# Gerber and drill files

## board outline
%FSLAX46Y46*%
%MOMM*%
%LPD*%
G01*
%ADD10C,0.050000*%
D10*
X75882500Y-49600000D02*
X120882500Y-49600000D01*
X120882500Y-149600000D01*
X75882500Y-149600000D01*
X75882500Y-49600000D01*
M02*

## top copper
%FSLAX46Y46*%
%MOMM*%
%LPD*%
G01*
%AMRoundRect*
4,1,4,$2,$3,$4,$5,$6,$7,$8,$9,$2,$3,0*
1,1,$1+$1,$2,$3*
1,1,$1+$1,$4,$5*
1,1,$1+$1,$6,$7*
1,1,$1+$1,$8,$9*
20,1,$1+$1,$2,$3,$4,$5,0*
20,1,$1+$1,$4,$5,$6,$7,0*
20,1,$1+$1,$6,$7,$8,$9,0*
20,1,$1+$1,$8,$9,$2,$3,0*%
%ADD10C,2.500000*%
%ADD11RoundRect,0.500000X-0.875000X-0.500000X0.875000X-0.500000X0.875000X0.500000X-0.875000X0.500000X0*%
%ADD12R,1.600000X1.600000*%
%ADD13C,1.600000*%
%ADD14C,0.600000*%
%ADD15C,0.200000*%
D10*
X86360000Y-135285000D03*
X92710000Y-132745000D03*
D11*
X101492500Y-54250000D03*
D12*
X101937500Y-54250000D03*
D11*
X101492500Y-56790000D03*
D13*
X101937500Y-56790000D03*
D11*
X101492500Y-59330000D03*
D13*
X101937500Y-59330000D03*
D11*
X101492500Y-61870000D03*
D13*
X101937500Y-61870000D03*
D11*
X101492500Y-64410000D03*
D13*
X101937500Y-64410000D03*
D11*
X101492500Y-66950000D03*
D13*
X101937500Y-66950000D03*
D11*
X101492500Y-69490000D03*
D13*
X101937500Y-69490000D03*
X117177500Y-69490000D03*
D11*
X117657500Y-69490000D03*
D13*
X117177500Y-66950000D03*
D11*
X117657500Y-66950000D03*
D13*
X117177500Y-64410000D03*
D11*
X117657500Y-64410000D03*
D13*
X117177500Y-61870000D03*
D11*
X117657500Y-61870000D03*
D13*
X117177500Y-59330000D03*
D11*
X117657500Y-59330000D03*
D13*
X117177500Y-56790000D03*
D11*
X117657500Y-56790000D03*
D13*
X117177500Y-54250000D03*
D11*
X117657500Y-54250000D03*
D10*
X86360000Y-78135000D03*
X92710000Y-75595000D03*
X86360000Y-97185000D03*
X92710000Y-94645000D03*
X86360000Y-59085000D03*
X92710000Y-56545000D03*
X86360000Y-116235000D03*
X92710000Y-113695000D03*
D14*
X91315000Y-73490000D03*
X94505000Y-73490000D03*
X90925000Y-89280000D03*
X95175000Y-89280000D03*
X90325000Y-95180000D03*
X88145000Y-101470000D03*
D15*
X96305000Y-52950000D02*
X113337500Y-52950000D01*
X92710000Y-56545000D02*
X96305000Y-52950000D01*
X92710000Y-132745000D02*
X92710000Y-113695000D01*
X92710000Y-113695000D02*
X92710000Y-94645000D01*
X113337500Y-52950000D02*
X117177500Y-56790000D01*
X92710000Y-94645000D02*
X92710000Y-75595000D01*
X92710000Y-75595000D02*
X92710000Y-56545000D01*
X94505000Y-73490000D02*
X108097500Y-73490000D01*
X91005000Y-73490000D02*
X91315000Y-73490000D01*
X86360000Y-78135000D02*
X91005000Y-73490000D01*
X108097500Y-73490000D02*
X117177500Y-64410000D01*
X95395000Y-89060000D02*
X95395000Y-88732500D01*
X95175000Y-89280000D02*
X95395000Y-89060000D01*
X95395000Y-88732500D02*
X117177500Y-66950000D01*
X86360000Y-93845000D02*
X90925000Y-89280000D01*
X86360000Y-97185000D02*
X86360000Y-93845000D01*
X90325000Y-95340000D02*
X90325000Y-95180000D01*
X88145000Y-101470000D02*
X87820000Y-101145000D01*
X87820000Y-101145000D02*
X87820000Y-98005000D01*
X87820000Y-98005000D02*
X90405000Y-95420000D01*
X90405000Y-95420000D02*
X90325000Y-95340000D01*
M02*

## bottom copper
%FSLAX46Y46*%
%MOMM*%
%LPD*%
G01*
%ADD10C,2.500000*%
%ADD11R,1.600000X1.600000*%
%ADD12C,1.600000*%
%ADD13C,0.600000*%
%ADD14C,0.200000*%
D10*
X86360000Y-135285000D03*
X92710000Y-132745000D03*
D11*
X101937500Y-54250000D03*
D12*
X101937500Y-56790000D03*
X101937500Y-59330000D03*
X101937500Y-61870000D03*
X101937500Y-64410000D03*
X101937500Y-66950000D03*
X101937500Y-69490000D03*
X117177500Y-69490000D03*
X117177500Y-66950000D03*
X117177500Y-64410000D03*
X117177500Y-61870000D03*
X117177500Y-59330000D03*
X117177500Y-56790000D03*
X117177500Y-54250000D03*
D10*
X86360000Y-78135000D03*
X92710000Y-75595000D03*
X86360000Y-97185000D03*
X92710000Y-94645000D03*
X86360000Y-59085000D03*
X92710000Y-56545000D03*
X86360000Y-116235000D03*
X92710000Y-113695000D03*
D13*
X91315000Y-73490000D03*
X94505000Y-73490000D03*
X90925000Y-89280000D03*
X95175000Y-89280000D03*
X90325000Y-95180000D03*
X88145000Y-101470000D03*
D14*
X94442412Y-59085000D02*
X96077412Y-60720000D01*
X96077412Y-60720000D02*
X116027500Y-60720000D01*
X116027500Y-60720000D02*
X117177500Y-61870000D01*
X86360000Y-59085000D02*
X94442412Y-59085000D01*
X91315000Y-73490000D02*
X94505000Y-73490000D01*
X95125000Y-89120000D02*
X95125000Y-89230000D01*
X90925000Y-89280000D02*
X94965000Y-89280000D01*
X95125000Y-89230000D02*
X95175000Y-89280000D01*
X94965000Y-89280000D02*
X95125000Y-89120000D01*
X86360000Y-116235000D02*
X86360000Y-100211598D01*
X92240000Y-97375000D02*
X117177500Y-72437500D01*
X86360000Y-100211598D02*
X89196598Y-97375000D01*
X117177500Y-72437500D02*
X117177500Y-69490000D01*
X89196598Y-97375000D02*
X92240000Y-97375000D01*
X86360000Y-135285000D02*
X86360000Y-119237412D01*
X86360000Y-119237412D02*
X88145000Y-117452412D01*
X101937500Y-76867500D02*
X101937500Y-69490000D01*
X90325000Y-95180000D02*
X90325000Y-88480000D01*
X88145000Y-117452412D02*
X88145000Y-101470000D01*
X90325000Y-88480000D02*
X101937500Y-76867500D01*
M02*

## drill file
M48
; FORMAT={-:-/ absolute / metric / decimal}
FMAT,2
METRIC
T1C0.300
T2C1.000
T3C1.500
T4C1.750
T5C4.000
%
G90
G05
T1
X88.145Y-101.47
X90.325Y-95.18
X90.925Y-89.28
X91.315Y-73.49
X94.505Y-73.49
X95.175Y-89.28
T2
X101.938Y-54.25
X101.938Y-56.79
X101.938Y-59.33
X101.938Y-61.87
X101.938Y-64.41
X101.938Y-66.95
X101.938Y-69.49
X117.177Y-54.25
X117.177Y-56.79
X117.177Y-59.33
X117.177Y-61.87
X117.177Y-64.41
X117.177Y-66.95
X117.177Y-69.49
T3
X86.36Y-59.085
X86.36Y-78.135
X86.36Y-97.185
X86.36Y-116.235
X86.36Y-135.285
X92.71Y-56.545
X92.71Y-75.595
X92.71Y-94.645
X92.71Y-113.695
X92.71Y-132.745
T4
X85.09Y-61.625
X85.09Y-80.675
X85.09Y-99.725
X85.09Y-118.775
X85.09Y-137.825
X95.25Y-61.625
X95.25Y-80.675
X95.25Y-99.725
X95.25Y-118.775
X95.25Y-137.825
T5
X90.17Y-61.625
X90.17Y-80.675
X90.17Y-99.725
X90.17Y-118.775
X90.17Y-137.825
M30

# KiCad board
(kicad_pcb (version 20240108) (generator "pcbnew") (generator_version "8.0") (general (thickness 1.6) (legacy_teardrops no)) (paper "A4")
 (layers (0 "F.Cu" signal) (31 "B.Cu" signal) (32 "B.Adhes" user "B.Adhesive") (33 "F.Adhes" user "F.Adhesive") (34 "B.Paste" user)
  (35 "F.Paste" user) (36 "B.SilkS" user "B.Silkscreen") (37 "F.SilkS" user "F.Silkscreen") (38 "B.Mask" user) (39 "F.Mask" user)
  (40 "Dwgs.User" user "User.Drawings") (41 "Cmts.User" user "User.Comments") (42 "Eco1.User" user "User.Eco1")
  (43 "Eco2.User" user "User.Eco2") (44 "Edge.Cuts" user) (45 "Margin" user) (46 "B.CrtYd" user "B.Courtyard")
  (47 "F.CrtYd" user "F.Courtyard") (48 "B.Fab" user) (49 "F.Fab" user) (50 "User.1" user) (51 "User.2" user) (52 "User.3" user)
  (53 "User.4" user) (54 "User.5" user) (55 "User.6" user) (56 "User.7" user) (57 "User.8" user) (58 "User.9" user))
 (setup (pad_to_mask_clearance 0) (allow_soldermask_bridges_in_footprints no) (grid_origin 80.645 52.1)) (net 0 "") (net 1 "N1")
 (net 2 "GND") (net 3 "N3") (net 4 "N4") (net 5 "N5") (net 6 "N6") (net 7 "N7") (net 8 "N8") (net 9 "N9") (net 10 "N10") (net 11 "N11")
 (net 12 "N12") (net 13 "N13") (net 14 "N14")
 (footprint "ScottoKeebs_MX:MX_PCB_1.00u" (layer "F.Cu") (at 90.17 137.825)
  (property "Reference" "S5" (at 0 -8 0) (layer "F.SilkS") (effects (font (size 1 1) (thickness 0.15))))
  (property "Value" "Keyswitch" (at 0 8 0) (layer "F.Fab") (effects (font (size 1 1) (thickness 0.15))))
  (pad "" np_thru_hole circle (at -5.08 0) (size 1.75 1.75) (drill 1.75) (layers "*.Cu" "*.Mask"))
  (pad "" np_thru_hole circle (at 0 0) (size 4 4) (drill 4) (layers "*.Cu" "*.Mask"))
  (pad "" np_thru_hole circle (at 5.08 0) (size 1.75 1.75) (drill 1.75) (layers "*.Cu" "*.Mask"))
  (pad "1" thru_hole circle (at -3.81 -2.54) (size 2.5 2.5) (drill 1.5) (layers "*.Cu" "*.Mask") (remove_unused_layers no) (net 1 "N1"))
  (pad "2" thru_hole circle (at 2.54 -5.08) (size 2.5 2.5) (drill 1.5) (layers "*.Cu" "*.Mask") (remove_unused_layers no) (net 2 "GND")))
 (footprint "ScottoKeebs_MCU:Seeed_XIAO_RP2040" (layer "F.Cu") (at 109.5575 61.87)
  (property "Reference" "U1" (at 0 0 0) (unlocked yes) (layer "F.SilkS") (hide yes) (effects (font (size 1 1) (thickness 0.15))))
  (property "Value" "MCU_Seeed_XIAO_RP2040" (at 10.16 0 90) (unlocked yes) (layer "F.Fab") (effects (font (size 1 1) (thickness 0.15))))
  (pad "1" smd roundrect (at -8.065 -7.62) (size 2.75 2) (layers "F.Cu" "F.Paste" "F.Mask") (roundrect_rratio 0.25) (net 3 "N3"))
  (pad "1" thru_hole rect (at -7.62 -7.62 90) (size 1.6 1.6) (drill 1) (layers "*.Cu" "*.Mask") (remove_unused_layers no) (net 3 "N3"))
  (pad "2" smd roundrect (at -8.065 -5.08) (size 2.75 2) (layers "F.Cu" "F.Paste" "F.Mask") (roundrect_rratio 0.25) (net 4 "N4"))
  (pad "2" thru_hole circle (at -7.62 -5.08 90) (size 1.6 1.6) (drill 1) (layers "*.Cu" "*.Mask") (remove_unused_layers no) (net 4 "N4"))
  (pad "3" smd roundrect (at -8.065 -2.54) (size 2.75 2) (layers "F.Cu" "F.Paste" "F.Mask") (roundrect_rratio 0.25) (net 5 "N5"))
  (pad "3" thru_hole circle (at -7.62 -2.54 90) (size 1.6 1.6) (drill 1) (layers "*.Cu" "*.Mask") (remove_unused_layers no) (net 5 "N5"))
  (pad "4" smd roundrect (at -8.065 0) (size 2.75 2) (layers "F.Cu" "F.Paste" "F.Mask") (roundrect_rratio 0.25) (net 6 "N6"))
  (pad "4" thru_hole circle (at -7.62 0 90) (size 1.6 1.6) (drill 1) (layers "*.Cu" "*.Mask") (remove_unused_layers no) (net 6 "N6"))
  (pad "5" smd roundrect (at -8.065 2.54) (size 2.75 2) (layers "F.Cu" "F.Paste" "F.Mask") (roundrect_rratio 0.25) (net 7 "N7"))
  (pad "5" thru_hole circle (at -7.62 2.54 90) (size 1.6 1.6) (drill 1) (layers "*.Cu" "*.Mask") (remove_unused_layers no) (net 7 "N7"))
  (pad "6" smd roundrect (at -8.065 5.08) (size 2.75 2) (layers "F.Cu" "F.Paste" "F.Mask") (roundrect_rratio 0.25) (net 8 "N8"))
  (pad "6" thru_hole circle (at -7.62 5.08 90) (size 1.6 1.6) (drill 1) (layers "*.Cu" "*.Mask") (remove_unused_layers no) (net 8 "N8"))
  (pad "7" smd roundrect (at -8.065 7.62) (size 2.75 2) (layers "F.Cu" "F.Paste" "F.Mask") (roundrect_rratio 0.25) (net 1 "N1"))
  (pad "7" thru_hole circle (at -7.62 7.62 90) (size 1.6 1.6) (drill 1) (layers "*.Cu" "*.Mask") (remove_unused_layers no) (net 1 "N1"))
  (pad "8" thru_hole circle (at 7.62 7.62 90) (size 1.6 1.6) (drill 1) (layers "*.Cu" "*.Mask") (remove_unused_layers no) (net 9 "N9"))
  (pad "8" smd roundrect (at 8.1 7.62) (size 2.75 2) (layers "F.Cu" "F.Paste" "F.Mask") (roundrect_rratio 0.25) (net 9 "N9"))
  (pad "9" thru_hole circle (at 7.62 5.08 90) (size 1.6 1.6) (drill 1) (layers "*.Cu" "*.Mask") (remove_unused_layers no) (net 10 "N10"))
  (pad "9" smd roundrect (at 8.1 5.08) (size 2.75 2) (layers "F.Cu" "F.Paste" "F.Mask") (roundrect_rratio 0.25) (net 10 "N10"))
  (pad "10" thru_hole circle (at 7.62 2.54 90) (size 1.6 1.6) (drill 1) (layers "*.Cu" "*.Mask") (remove_unused_layers no) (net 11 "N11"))
  (pad "10" smd roundrect (at 8.1 2.54) (size 2.75 2) (layers "F.Cu" "F.Paste" "F.Mask") (roundrect_rratio 0.25) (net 11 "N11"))
  (pad "11" thru_hole circle (at 7.62 0 90) (size 1.6 1.6) (drill 1) (layers "*.Cu" "*.Mask") (remove_unused_layers no) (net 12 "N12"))
  (pad "11" smd roundrect (at 8.1 0) (size 2.75 2) (layers "F.Cu" "F.Paste" "F.Mask") (roundrect_rratio 0.25) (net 12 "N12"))
  (pad "12" thru_hole circle (at 7.62 -2.54 90) (size 1.6 1.6) (drill 1) (layers "*.Cu" "*.Mask") (remove_unused_layers no) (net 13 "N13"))
  (pad "12" smd roundrect (at 8.1 -2.54) (size 2.75 2) (layers "F.Cu" "F.Paste" "F.Mask") (roundrect_rratio 0.25) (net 13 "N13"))
  (pad "13" thru_hole circle (at 7.62 -5.08 90) (size 1.6 1.6) (drill 1) (layers "*.Cu" "*.Mask") (remove_unused_layers no) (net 2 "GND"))
  (pad "13" smd roundrect (at 8.1 -5.08) (size 2.75 2) (layers "F.Cu" "F.Paste" "F.Mask") (roundrect_rratio 0.25) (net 2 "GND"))
  (pad "14" thru_hole circle (at 7.62 -7.62 90) (size 1.6 1.6) (drill 1) (layers "*.Cu" "*.Mask") (remove_unused_layers no) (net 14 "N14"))
  (pad "14" smd roundrect (at 8.1 -7.62) (size 2.75 2) (layers "F.Cu" "F.Paste" "F.Mask") (roundrect_rratio 0.25) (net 14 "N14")))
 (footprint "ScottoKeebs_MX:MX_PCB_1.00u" (layer "F.Cu") (at 90.17 80.675)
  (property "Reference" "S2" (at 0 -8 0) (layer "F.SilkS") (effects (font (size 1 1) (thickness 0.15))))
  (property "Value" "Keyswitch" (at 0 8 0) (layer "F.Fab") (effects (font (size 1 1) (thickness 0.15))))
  (pad "" np_thru_hole circle (at -5.08 0) (size 1.75 1.75) (drill 1.75) (layers "*.Cu" "*.Mask"))
  (pad "" np_thru_hole circle (at 0 0) (size 4 4) (drill 4) (layers "*.Cu" "*.Mask"))
  (pad "" np_thru_hole circle (at 5.08 0) (size 1.75 1.75) (drill 1.75) (layers "*.Cu" "*.Mask"))
  (pad "1" thru_hole circle (at -3.81 -2.54) (size 2.5 2.5) (drill 1.5) (layers "*.Cu" "*.Mask") (remove_unused_layers no) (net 11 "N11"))
  (pad "2" thru_hole circle (at 2.54 -5.08) (size 2.5 2.5) (drill 1.5) (layers "*.Cu" "*.Mask") (remove_unused_layers no) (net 2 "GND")))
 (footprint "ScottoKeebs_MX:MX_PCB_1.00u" (layer "F.Cu") (at 90.17 99.725)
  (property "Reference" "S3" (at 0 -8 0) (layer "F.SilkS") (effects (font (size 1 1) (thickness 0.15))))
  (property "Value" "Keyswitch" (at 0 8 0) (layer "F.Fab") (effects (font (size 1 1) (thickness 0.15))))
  (pad "" np_thru_hole circle (at -5.08 0) (size 1.75 1.75) (drill 1.75) (layers "*.Cu" "*.Mask"))
  (pad "" np_thru_hole circle (at 0 0) (size 4 4) (drill 4) (layers "*.Cu" "*.Mask"))
  (pad "" np_thru_hole circle (at 5.08 0) (size 1.75 1.75) (drill 1.75) (layers "*.Cu" "*.Mask"))
  (pad "1" thru_hole circle (at -3.81 -2.54) (size 2.5 2.5) (drill 1.5) (layers "*.Cu" "*.Mask") (remove_unused_layers no) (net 10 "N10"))
  (pad "2" thru_hole circle (at 2.54 -5.08) (size 2.5 2.5) (drill 1.5) (layers "*.Cu" "*.Mask") (remove_unused_layers no) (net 2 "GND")))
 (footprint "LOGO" (layer "F.Cu") (at 116.71771 92.292004 -90)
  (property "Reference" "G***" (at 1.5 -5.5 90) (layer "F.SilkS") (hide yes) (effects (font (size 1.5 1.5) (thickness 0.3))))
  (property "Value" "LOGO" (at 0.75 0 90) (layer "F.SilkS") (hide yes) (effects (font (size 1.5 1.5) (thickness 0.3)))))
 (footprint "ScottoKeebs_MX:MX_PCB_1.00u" (layer "F.Cu") (at 90.17 61.625)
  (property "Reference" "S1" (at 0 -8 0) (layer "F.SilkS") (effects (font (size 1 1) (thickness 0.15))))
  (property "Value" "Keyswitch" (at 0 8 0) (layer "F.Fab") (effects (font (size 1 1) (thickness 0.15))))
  (pad "" np_thru_hole circle (at -5.08 0) (size 1.75 1.75) (drill 1.75) (layers "*.Cu" "*.Mask"))
  (pad "" np_thru_hole circle (at 0 0) (size 4 4) (drill 4) (layers "*.Cu" "*.Mask"))
  (pad "" np_thru_hole circle (at 5.08 0) (size 1.75 1.75) (drill 1.75) (layers "*.Cu" "*.Mask"))
  (pad "1" thru_hole circle (at -3.81 -2.54) (size 2.5 2.5) (drill 1.5) (layers "*.Cu" "*.Mask") (remove_unused_layers no) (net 12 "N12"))
  (pad "2" thru_hole circle (at 2.54 -5.08) (size 2.5 2.5) (drill 1.5) (layers "*.Cu" "*.Mask") (remove_unused_layers no) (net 2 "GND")))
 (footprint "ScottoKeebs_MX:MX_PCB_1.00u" (layer "F.Cu") (at 90.17 118.775)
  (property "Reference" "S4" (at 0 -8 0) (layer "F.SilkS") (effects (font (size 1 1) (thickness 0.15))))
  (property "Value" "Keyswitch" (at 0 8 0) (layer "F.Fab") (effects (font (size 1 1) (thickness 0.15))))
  (pad "" np_thru_hole circle (at -5.08 0) (size 1.75 1.75) (drill 1.75) (layers "*.Cu" "*.Mask"))
  (pad "" np_thru_hole circle (at 0 0) (size 4 4) (drill 4) (layers "*.Cu" "*.Mask"))
  (pad "" np_thru_hole circle (at 5.08 0) (size 1.75 1.75) (drill 1.75) (layers "*.Cu" "*.Mask"))
  (pad "1" thru_hole circle (at -3.81 -2.54) (size 2.5 2.5) (drill 1.5) (layers "*.Cu" "*.Mask") (remove_unused_layers no) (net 9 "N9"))
  (pad "2" thru_hole circle (at 2.54 -5.08) (size 2.5 2.5) (drill 1.5) (layers "*.Cu" "*.Mask") (remove_unused_layers no) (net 2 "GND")))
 (gr_rect (start 75.8825 49.6) (end 120.8825 149.6) (stroke (width 0.05) (type default)) (fill none) (layer "Edge.Cuts"))
 (segment (start 96.305 52.95) (end 113.3375 52.95) (width 0.2) (layer "F.Cu") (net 2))
 (segment (start 92.71 56.545) (end 96.305 52.95) (width 0.2) (layer "F.Cu") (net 2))
 (segment (start 92.71 132.745) (end 92.71 113.695) (width 0.2) (layer "F.Cu") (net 2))
 (segment (start 92.71 113.695) (end 92.71 94.645) (width 0.2) (layer "F.Cu") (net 2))
 (segment (start 113.3375 52.95) (end 117.1775 56.79) (width 0.2) (layer "F.Cu") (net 2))
 (segment (start 92.71 94.645) (end 92.71 75.595) (width 0.2) (layer "F.Cu") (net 2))
 (segment (start 92.71 75.595) (end 92.71 56.545) (width 0.2) (layer "F.Cu") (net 2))
 (segment (start 94.442412 59.085) (end 96.077412 60.72) (width 0.2) (layer "B.Cu") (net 12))
 (segment (start 96.077412 60.72) (end 116.0275 60.72) (width 0.2) (layer "B.Cu") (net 12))
 (segment (start 116.0275 60.72) (end 117.1775 61.87) (width 0.2) (layer "B.Cu") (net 12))
 (segment (start 86.36 59.085) (end 94.442412 59.085) (width 0.2) (layer "B.Cu") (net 12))
 (segment (start 94.505 73.49) (end 108.0975 73.49) (width 0.2) (layer "F.Cu") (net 11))
 (segment (start 91.005 73.49) (end 91.315 73.49) (width 0.2) (layer "F.Cu") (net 11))
 (segment (start 86.36 78.135) (end 91.005 73.49) (width 0.2) (layer "F.Cu") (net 11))
 (segment (start 108.0975 73.49) (end 117.1775 64.41) (width 0.2) (layer "F.Cu") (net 11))
 (via (at 91.315 73.49) (size 0.6) (drill 0.3) (layers "F.Cu" "B.Cu") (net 11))
 (via (at 94.505 73.49) (size 0.6) (drill 0.3) (layers "F.Cu" "B.Cu") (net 11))
 (segment (start 91.315 73.49) (end 94.505 73.49) (width 0.2) (layer "B.Cu") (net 11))
 (segment (start 95.395 89.06) (end 95.395 88.7325) (width 0.2) (layer "F.Cu") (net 10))
 (segment (start 95.175 89.28) (end 95.395 89.06) (width 0.2) (layer "F.Cu") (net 10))
 (segment (start 95.395 88.7325) (end 117.1775 66.95) (width 0.2) (layer "F.Cu") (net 10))
 (segment (start 86.36 93.845) (end 90.925 89.28) (width 0.2) (layer "F.Cu") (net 10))
 (segment (start 86.36 97.185) (end 86.36 93.845) (width 0.2) (layer "F.Cu") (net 10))
 (via (at 90.925 89.28) (size 0.6) (drill 0.3) (layers "F.Cu" "B.Cu") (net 10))
 (via (at 95.175 89.28) (size 0.6) (drill 0.3) (layers "F.Cu" "B.Cu") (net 10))
 (segment (start 95.125 89.12) (end 95.125 89.23) (width 0.2) (layer "B.Cu") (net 10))
 (segment (start 90.925 89.28) (end 94.965 89.28) (width 0.2) (layer "B.Cu") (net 10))
 (segment (start 95.125 89.23) (end 95.175 89.28) (width 0.2) (layer "B.Cu") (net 10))
 (segment (start 94.965 89.28) (end 95.125 89.12) (width 0.2) (layer "B.Cu") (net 10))
 (segment (start 86.36 116.235) (end 86.36 100.211598) (width 0.2) (layer "B.Cu") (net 9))
 (segment (start 92.24 97.375) (end 117.1775 72.4375) (width 0.2) (layer "B.Cu") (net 9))
 (segment (start 86.36 100.211598) (end 89.196598 97.375) (width 0.2) (layer "B.Cu") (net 9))
 (segment (start 117.1775 72.4375) (end 117.1775 69.49) (width 0.2) (layer "B.Cu") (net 9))
 (segment (start 89.196598 97.375) (end 92.24 97.375) (width 0.2) (layer "B.Cu") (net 9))
 (segment (start 90.325 95.34) (end 90.325 95.18) (width 0.2) (layer "F.Cu") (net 1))
 (segment (start 88.145 101.47) (end 87.82 101.145) (width 0.2) (layer "F.Cu") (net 1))
 (segment (start 87.82 101.145) (end 87.82 98.005) (width 0.2) (layer "F.Cu") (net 1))
 (segment (start 87.82 98.005) (end 90.405 95.42) (width 0.2) (layer "F.Cu") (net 1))
 (segment (start 90.405 95.42) (end 90.325 95.34) (width 0.2) (layer "F.Cu") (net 1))
 (via (at 90.325 95.18) (size 0.6) (drill 0.3) (layers "F.Cu" "B.Cu") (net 1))
 (via (at 88.145 101.47) (size 0.6) (drill 0.3) (layers "F.Cu" "B.Cu") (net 1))
 (segment (start 86.36 135.285) (end 86.36 119.237412) (width 0.2) (layer "B.Cu") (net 1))
 (segment (start 86.36 119.237412) (end 88.145 117.452412) (width 0.2) (layer "B.Cu") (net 1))
 (segment (start 101.9375 76.8675) (end 101.9375 69.49) (width 0.2) (layer "B.Cu") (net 1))
 (segment (start 90.325 95.18) (end 90.325 88.48) (width 0.2) (layer "B.Cu") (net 1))
 (segment (start 88.145 117.452412) (end 88.145 101.47) (width 0.2) (layer "B.Cu") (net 1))
 (segment (start 90.325 88.48) (end 101.9375 76.8675) (width 0.2) (layer "B.Cu") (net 1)))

